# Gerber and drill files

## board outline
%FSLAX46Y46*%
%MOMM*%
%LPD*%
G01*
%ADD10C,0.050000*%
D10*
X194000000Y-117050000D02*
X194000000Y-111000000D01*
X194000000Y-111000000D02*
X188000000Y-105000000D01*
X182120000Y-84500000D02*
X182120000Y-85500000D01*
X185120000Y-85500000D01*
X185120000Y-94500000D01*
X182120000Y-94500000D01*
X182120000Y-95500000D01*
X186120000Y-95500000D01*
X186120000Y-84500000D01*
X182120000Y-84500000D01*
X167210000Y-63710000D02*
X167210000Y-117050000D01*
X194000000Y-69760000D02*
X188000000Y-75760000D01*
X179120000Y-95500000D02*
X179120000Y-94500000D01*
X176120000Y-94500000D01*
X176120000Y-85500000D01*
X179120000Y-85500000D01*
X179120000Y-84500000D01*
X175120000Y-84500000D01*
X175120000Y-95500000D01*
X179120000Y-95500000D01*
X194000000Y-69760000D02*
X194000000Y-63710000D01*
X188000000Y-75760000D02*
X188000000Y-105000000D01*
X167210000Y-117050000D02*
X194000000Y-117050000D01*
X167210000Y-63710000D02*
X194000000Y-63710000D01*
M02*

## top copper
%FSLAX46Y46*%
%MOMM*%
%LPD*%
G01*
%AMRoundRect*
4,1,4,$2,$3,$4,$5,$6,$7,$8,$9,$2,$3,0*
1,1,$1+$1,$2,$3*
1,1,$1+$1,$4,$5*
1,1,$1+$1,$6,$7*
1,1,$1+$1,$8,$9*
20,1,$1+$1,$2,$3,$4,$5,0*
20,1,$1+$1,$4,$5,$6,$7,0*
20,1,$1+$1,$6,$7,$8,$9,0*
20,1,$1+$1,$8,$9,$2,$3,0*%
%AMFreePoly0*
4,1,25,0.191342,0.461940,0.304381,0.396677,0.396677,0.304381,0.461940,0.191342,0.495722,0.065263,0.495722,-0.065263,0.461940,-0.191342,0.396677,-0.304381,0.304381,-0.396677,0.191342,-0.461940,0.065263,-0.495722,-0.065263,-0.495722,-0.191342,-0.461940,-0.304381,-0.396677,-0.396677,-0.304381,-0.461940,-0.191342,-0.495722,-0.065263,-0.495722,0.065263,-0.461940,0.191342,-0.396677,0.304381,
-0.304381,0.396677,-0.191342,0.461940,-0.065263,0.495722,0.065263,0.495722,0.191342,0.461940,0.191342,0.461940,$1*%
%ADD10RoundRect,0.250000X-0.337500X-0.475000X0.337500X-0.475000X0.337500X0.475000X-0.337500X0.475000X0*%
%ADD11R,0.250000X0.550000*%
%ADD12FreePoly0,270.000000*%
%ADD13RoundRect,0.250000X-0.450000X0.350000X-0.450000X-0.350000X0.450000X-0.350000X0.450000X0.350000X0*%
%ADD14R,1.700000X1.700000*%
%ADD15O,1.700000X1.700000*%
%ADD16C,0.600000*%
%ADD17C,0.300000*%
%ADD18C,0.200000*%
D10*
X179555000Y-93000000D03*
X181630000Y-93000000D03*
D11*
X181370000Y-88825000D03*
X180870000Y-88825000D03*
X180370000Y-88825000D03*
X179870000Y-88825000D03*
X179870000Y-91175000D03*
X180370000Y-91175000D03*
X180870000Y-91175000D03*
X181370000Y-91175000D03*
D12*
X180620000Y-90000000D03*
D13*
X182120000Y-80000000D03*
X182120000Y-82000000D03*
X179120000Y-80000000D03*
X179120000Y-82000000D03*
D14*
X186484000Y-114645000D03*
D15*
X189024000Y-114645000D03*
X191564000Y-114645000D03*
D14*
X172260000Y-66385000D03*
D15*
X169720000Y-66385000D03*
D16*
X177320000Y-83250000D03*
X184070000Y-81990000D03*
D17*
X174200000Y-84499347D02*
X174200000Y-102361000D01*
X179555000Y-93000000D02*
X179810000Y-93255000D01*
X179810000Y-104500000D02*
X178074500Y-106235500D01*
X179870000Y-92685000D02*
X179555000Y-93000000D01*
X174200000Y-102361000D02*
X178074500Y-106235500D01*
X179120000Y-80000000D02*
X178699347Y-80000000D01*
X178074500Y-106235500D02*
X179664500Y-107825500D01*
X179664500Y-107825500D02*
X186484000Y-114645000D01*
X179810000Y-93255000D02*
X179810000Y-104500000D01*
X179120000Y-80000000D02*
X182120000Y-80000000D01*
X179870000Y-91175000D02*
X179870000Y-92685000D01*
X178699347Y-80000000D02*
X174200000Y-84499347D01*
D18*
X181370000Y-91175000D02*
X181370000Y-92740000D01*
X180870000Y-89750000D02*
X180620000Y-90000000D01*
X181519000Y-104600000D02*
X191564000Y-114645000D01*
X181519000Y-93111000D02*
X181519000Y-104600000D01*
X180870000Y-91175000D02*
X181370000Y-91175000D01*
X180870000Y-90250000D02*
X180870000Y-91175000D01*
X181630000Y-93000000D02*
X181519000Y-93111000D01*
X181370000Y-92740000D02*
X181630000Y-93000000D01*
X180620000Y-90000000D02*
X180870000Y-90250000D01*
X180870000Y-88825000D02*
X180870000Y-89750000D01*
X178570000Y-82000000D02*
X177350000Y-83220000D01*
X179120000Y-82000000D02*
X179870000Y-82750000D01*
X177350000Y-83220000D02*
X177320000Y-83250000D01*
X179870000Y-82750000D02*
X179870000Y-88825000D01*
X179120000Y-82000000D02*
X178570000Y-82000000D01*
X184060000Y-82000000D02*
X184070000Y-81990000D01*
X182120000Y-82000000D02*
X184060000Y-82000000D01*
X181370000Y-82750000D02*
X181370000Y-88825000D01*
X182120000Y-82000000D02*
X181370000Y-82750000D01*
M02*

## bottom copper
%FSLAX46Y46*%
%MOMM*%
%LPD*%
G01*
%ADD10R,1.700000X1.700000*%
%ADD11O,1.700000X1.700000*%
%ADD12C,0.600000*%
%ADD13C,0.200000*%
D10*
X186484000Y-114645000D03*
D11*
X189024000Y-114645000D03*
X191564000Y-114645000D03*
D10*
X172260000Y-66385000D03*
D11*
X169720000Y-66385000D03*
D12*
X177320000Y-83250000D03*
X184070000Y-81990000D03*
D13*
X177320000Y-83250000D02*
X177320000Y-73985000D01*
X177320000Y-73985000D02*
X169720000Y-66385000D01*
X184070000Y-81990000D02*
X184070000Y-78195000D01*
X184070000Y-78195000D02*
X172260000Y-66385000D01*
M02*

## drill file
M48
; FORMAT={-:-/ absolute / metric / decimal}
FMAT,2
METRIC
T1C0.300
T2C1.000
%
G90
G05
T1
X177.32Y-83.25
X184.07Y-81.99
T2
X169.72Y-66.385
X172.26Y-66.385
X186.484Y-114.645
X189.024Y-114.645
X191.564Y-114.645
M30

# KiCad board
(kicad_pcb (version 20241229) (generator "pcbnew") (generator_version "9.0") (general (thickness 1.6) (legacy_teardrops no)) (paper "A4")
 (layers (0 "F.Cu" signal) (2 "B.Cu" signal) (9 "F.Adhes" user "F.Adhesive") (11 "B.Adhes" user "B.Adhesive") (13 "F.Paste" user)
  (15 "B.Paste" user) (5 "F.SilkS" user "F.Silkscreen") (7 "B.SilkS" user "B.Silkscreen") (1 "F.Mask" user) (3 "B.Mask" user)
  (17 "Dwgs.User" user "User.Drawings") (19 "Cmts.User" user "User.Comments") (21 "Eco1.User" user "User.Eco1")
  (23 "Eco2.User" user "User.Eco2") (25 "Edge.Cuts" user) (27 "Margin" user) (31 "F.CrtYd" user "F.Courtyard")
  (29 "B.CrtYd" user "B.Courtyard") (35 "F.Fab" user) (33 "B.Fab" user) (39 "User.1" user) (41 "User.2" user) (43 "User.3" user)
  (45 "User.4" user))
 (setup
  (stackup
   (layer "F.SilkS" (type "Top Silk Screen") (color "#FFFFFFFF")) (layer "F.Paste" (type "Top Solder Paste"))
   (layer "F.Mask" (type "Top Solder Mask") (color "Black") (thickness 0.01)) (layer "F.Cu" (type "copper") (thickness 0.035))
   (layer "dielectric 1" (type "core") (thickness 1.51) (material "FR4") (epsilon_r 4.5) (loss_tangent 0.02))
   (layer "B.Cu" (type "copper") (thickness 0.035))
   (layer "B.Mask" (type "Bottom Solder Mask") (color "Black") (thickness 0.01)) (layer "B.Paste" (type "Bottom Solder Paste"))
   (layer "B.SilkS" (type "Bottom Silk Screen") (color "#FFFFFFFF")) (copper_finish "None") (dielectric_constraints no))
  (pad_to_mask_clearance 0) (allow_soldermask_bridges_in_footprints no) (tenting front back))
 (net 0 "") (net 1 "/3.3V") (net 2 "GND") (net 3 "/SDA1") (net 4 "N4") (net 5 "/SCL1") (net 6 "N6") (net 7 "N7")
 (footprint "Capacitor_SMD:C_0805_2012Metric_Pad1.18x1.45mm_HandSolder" (layer "F.Cu") (at 180.5925 93)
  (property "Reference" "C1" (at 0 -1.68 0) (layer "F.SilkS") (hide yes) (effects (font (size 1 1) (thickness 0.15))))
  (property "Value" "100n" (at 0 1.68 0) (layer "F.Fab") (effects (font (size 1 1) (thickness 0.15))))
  (pad "1" smd roundrect (at -1.0375 0) (size 1.175 1.45) (layers "F.Cu" "F.Mask" "F.Paste") (roundrect_rratio 0.212766) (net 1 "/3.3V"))
  (pad "2" smd roundrect (at 1.0375 0) (size 1.175 1.45) (layers "F.Cu" "F.Mask" "F.Paste") (roundrect_rratio 0.212766) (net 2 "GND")))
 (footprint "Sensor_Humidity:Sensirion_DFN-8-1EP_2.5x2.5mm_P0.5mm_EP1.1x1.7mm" (layer "F.Cu") (at 180.62 90 -90)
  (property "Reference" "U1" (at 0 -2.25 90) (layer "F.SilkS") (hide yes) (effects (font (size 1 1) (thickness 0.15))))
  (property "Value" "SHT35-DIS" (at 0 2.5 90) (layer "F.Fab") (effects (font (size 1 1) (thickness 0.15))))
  (pad "" smd custom (at 0 0 270) (size 0.9 0.9) (layers "F.Paste") (zone_connect 0) (thermal_bridge_angle 45)
   (options (clearance outline) (anchor rect)) (primitives))
  (pad "1" smd rect (at -1.175 -0.75 270) (size 0.55 0.25) (layers "F.Cu" "F.Mask" "F.Paste") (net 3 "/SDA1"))
  (pad "2" smd rect (at -1.175 -0.25 270) (size 0.55 0.25) (layers "F.Cu" "F.Mask" "F.Paste") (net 2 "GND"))
  (pad "3" smd rect (at -1.175 0.25 270) (size 0.55 0.25) (layers "F.Cu" "F.Mask" "F.Paste") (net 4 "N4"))
  (pad "4" smd rect (at -1.175 0.75 90) (size 0.55 0.25) (layers "F.Cu" "F.Mask" "F.Paste") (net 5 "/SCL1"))
  (pad "5" smd rect (at 1.175 0.75 270) (size 0.55 0.25) (layers "F.Cu" "F.Mask" "F.Paste") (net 1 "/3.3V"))
  (pad "6" smd rect (at 1.175 0.25 270) (size 0.55 0.25) (layers "F.Cu" "F.Mask" "F.Paste") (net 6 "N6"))
  (pad "7" smd rect (at 1.175 -0.25 270) (size 0.55 0.25) (layers "F.Cu" "F.Mask" "F.Paste") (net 2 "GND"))
  (pad "8" smd rect (at 1.175 -0.75 270) (size 0.55 0.25) (layers "F.Cu" "F.Mask" "F.Paste") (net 2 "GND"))
  (pad "9" smd custom (at 0 0 270) (size 1 1) (layers "F.Cu" "F.Mask") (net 2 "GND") (zone_connect 0)
   (options (clearance outline) (anchor circle)) (primitives)))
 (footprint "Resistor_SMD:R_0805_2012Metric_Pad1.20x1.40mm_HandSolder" (layer "F.Cu") (at 182.12 81 -90)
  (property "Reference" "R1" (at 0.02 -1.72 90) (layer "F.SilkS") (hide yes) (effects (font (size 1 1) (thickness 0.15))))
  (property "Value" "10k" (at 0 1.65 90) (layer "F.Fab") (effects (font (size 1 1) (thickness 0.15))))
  (pad "1" smd roundrect (at -1 0 270) (size 1.2 1.4) (layers "F.Cu" "F.Mask" "F.Paste") (roundrect_rratio 0.208333) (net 1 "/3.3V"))
  (pad "2" smd roundrect (at 1 0 270) (size 1.2 1.4) (layers "F.Cu" "F.Mask" "F.Paste") (roundrect_rratio 0.208333) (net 3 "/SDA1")))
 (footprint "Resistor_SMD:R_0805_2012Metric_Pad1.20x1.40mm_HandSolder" (layer "F.Cu") (at 179.12 81 -90)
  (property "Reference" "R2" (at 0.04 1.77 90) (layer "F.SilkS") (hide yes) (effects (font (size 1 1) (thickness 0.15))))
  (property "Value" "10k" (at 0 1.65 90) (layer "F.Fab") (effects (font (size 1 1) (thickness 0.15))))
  (pad "1" smd roundrect (at -1 0 270) (size 1.2 1.4) (layers "F.Cu" "F.Mask" "F.Paste") (roundrect_rratio 0.208333) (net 1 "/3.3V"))
  (pad "2" smd roundrect (at 1 0 270) (size 1.2 1.4) (layers "F.Cu" "F.Mask" "F.Paste") (roundrect_rratio 0.208333) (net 5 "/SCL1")))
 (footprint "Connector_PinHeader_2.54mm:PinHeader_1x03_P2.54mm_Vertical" (layer "B.Cu") (at 186.484 114.645 -90)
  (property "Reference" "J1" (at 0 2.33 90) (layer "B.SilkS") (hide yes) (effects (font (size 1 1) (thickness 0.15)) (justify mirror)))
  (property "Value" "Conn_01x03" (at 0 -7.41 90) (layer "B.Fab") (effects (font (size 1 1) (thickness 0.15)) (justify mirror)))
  (pad "1" thru_hole rect (at 0 0 270) (size 1.7 1.7) (drill 1) (layers "*.Cu" "*.Mask") (remove_unused_layers no) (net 1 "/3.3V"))
  (pad "2" thru_hole oval (at 0 -2.54 270) (size 1.7 1.7) (drill 1) (layers "*.Cu" "*.Mask") (remove_unused_layers no) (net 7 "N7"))
  (pad "3" thru_hole oval (at 0 -5.08 270) (size 1.7 1.7) (drill 1) (layers "*.Cu" "*.Mask") (remove_unused_layers no) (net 2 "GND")))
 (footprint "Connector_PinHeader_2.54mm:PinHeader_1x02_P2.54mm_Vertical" (layer "B.Cu") (at 172.26 66.385 90)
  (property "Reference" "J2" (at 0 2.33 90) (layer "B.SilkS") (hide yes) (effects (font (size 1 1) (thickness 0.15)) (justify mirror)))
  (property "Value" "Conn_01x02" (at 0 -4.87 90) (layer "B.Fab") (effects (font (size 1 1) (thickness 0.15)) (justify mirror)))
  (pad "1" thru_hole rect (at 0 0 90) (size 1.7 1.7) (drill 1) (layers "*.Cu" "*.Mask") (remove_unused_layers no) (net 3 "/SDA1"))
  (pad "2" thru_hole oval (at 0 -2.54 90) (size 1.7 1.7) (drill 1) (layers "*.Cu" "*.Mask") (remove_unused_layers no) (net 5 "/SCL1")))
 (gr_line (start 194 117.05) (end 194 111) (stroke (width 0.05) (type default)) (layer "Edge.Cuts"))
 (gr_line (start 194 111) (end 188 105) (stroke (width 0.05) (type default)) (layer "Edge.Cuts"))
 (gr_poly
  (pts (xy 182.12 84.5) (xy 182.12 85.5) (xy 185.12 85.5) (xy 185.12 94.5) (xy 182.12 94.5) (xy 182.12 95.5) (xy 186.12 95.5)
   (xy 186.12 84.5))
  (stroke (width 0.05) (type solid)) (fill no) (layer "Edge.Cuts"))
 (gr_line (start 167.21 63.71) (end 167.21 117.05) (stroke (width 0.05) (type default)) (layer "Edge.Cuts"))
 (gr_line (start 194 69.76) (end 188 75.76) (stroke (width 0.05) (type default)) (layer "Edge.Cuts"))
 (gr_poly
  (pts (xy 179.12 95.5) (xy 179.12 94.5) (xy 176.12 94.5) (xy 176.12 85.5) (xy 179.12 85.5) (xy 179.12 84.5) (xy 175.12 84.5)
   (xy 175.12 95.5))
  (stroke (width 0.05) (type solid)) (fill no) (layer "Edge.Cuts"))
 (gr_line (start 194 69.76) (end 194 63.71) (stroke (width 0.05) (type default)) (layer "Edge.Cuts"))
 (gr_line (start 188 75.76) (end 188 105) (stroke (width 0.05) (type default)) (layer "Edge.Cuts"))
 (gr_line (start 167.21 117.05) (end 194 117.05) (stroke (width 0.05) (type default)) (layer "Edge.Cuts"))
 (gr_line (start 167.21 63.71) (end 194 63.71) (stroke (width 0.05) (type default)) (layer "Edge.Cuts"))
 (segment (start 174.2 84.499347) (end 174.2 102.361) (width 0.3) (layer "F.Cu") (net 1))
 (segment (start 179.555 93) (end 179.81 93.255) (width 0.3) (layer "F.Cu") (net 1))
 (segment (start 179.81 104.5) (end 178.0745 106.2355) (width 0.3) (layer "F.Cu") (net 1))
 (segment (start 179.87 92.685) (end 179.555 93) (width 0.3) (layer "F.Cu") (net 1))
 (segment (start 174.2 102.361) (end 178.0745 106.2355) (width 0.3) (layer "F.Cu") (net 1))
 (segment (start 179.12 80) (end 178.699347 80) (width 0.3) (layer "F.Cu") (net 1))
 (segment (start 178.0745 106.2355) (end 179.6645 107.8255) (width 0.3) (layer "F.Cu") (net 1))
 (segment (start 179.6645 107.8255) (end 186.484 114.645) (width 0.3) (layer "F.Cu") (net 1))
 (segment (start 179.81 93.255) (end 179.81 104.5) (width 0.3) (layer "F.Cu") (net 1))
 (segment (start 179.12 80) (end 182.12 80) (width 0.3) (layer "F.Cu") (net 1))
 (segment (start 179.87 91.175) (end 179.87 92.685) (width 0.3) (layer "F.Cu") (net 1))
 (segment (start 178.699347 80) (end 174.2 84.499347) (width 0.3) (layer "F.Cu") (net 1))
 (segment (start 181.37 91.175) (end 181.37 92.74) (width 0.2) (layer "F.Cu") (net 2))
 (segment (start 180.87 89.75) (end 180.62 90) (width 0.2) (layer "F.Cu") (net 2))
 (segment (start 181.519 104.6) (end 191.564 114.645) (width 0.2) (layer "F.Cu") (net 2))
 (segment (start 181.519 93.111) (end 181.519 104.6) (width 0.2) (layer "F.Cu") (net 2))
 (segment (start 180.87 91.175) (end 181.37 91.175) (width 0.2) (layer "F.Cu") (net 2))
 (segment (start 180.87 90.25) (end 180.87 91.175) (width 0.2) (layer "F.Cu") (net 2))
 (segment (start 181.63 93) (end 181.519 93.111) (width 0.2) (layer "F.Cu") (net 2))
 (segment (start 181.37 92.74) (end 181.63 93) (width 0.2) (layer "F.Cu") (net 2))
 (segment (start 180.62 90) (end 180.87 90.25) (width 0.2) (layer "F.Cu") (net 2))
 (segment (start 180.87 88.825) (end 180.87 89.75) (width 0.2) (layer "F.Cu") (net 2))
 (segment (start 178.57 82) (end 177.35 83.22) (width 0.2) (layer "F.Cu") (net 5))
 (segment (start 179.12 82) (end 179.87 82.75) (width 0.2) (layer "F.Cu") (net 5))
 (segment (start 177.35 83.22) (end 177.32 83.25) (width 0.2) (layer "F.Cu") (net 5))
 (segment (start 179.87 82.75) (end 179.87 88.825) (width 0.2) (layer "F.Cu") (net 5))
 (segment (start 179.12 82) (end 178.57 82) (width 0.2) (layer "F.Cu") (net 5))
 (via (at 177.32 83.25) (size 0.6) (drill 0.3) (layers "F.Cu" "B.Cu") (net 5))
 (segment (start 177.32 83.25) (end 177.32 73.985) (width 0.2) (layer "B.Cu") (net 5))
 (segment (start 177.32 73.985) (end 169.72 66.385) (width 0.2) (layer "B.Cu") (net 5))
 (segment (start 184.06 82) (end 184.07 81.99) (width 0.2) (layer "F.Cu") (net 3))
 (segment (start 182.12 82) (end 184.06 82) (width 0.2) (layer "F.Cu") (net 3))
 (segment (start 181.37 82.75) (end 181.37 88.825) (width 0.2) (layer "F.Cu") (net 3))
 (segment (start 182.12 82) (end 181.37 82.75) (width 0.2) (layer "F.Cu") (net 3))
 (via (at 184.07 81.99) (size 0.6) (drill 0.3) (layers "F.Cu" "B.Cu") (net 3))
 (segment (start 184.07 81.99) (end 184.07 78.195) (width 0.2) (layer "B.Cu") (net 3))
 (segment (start 184.07 78.195) (end 172.26 66.385) (width 0.2) (layer "B.Cu") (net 3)))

